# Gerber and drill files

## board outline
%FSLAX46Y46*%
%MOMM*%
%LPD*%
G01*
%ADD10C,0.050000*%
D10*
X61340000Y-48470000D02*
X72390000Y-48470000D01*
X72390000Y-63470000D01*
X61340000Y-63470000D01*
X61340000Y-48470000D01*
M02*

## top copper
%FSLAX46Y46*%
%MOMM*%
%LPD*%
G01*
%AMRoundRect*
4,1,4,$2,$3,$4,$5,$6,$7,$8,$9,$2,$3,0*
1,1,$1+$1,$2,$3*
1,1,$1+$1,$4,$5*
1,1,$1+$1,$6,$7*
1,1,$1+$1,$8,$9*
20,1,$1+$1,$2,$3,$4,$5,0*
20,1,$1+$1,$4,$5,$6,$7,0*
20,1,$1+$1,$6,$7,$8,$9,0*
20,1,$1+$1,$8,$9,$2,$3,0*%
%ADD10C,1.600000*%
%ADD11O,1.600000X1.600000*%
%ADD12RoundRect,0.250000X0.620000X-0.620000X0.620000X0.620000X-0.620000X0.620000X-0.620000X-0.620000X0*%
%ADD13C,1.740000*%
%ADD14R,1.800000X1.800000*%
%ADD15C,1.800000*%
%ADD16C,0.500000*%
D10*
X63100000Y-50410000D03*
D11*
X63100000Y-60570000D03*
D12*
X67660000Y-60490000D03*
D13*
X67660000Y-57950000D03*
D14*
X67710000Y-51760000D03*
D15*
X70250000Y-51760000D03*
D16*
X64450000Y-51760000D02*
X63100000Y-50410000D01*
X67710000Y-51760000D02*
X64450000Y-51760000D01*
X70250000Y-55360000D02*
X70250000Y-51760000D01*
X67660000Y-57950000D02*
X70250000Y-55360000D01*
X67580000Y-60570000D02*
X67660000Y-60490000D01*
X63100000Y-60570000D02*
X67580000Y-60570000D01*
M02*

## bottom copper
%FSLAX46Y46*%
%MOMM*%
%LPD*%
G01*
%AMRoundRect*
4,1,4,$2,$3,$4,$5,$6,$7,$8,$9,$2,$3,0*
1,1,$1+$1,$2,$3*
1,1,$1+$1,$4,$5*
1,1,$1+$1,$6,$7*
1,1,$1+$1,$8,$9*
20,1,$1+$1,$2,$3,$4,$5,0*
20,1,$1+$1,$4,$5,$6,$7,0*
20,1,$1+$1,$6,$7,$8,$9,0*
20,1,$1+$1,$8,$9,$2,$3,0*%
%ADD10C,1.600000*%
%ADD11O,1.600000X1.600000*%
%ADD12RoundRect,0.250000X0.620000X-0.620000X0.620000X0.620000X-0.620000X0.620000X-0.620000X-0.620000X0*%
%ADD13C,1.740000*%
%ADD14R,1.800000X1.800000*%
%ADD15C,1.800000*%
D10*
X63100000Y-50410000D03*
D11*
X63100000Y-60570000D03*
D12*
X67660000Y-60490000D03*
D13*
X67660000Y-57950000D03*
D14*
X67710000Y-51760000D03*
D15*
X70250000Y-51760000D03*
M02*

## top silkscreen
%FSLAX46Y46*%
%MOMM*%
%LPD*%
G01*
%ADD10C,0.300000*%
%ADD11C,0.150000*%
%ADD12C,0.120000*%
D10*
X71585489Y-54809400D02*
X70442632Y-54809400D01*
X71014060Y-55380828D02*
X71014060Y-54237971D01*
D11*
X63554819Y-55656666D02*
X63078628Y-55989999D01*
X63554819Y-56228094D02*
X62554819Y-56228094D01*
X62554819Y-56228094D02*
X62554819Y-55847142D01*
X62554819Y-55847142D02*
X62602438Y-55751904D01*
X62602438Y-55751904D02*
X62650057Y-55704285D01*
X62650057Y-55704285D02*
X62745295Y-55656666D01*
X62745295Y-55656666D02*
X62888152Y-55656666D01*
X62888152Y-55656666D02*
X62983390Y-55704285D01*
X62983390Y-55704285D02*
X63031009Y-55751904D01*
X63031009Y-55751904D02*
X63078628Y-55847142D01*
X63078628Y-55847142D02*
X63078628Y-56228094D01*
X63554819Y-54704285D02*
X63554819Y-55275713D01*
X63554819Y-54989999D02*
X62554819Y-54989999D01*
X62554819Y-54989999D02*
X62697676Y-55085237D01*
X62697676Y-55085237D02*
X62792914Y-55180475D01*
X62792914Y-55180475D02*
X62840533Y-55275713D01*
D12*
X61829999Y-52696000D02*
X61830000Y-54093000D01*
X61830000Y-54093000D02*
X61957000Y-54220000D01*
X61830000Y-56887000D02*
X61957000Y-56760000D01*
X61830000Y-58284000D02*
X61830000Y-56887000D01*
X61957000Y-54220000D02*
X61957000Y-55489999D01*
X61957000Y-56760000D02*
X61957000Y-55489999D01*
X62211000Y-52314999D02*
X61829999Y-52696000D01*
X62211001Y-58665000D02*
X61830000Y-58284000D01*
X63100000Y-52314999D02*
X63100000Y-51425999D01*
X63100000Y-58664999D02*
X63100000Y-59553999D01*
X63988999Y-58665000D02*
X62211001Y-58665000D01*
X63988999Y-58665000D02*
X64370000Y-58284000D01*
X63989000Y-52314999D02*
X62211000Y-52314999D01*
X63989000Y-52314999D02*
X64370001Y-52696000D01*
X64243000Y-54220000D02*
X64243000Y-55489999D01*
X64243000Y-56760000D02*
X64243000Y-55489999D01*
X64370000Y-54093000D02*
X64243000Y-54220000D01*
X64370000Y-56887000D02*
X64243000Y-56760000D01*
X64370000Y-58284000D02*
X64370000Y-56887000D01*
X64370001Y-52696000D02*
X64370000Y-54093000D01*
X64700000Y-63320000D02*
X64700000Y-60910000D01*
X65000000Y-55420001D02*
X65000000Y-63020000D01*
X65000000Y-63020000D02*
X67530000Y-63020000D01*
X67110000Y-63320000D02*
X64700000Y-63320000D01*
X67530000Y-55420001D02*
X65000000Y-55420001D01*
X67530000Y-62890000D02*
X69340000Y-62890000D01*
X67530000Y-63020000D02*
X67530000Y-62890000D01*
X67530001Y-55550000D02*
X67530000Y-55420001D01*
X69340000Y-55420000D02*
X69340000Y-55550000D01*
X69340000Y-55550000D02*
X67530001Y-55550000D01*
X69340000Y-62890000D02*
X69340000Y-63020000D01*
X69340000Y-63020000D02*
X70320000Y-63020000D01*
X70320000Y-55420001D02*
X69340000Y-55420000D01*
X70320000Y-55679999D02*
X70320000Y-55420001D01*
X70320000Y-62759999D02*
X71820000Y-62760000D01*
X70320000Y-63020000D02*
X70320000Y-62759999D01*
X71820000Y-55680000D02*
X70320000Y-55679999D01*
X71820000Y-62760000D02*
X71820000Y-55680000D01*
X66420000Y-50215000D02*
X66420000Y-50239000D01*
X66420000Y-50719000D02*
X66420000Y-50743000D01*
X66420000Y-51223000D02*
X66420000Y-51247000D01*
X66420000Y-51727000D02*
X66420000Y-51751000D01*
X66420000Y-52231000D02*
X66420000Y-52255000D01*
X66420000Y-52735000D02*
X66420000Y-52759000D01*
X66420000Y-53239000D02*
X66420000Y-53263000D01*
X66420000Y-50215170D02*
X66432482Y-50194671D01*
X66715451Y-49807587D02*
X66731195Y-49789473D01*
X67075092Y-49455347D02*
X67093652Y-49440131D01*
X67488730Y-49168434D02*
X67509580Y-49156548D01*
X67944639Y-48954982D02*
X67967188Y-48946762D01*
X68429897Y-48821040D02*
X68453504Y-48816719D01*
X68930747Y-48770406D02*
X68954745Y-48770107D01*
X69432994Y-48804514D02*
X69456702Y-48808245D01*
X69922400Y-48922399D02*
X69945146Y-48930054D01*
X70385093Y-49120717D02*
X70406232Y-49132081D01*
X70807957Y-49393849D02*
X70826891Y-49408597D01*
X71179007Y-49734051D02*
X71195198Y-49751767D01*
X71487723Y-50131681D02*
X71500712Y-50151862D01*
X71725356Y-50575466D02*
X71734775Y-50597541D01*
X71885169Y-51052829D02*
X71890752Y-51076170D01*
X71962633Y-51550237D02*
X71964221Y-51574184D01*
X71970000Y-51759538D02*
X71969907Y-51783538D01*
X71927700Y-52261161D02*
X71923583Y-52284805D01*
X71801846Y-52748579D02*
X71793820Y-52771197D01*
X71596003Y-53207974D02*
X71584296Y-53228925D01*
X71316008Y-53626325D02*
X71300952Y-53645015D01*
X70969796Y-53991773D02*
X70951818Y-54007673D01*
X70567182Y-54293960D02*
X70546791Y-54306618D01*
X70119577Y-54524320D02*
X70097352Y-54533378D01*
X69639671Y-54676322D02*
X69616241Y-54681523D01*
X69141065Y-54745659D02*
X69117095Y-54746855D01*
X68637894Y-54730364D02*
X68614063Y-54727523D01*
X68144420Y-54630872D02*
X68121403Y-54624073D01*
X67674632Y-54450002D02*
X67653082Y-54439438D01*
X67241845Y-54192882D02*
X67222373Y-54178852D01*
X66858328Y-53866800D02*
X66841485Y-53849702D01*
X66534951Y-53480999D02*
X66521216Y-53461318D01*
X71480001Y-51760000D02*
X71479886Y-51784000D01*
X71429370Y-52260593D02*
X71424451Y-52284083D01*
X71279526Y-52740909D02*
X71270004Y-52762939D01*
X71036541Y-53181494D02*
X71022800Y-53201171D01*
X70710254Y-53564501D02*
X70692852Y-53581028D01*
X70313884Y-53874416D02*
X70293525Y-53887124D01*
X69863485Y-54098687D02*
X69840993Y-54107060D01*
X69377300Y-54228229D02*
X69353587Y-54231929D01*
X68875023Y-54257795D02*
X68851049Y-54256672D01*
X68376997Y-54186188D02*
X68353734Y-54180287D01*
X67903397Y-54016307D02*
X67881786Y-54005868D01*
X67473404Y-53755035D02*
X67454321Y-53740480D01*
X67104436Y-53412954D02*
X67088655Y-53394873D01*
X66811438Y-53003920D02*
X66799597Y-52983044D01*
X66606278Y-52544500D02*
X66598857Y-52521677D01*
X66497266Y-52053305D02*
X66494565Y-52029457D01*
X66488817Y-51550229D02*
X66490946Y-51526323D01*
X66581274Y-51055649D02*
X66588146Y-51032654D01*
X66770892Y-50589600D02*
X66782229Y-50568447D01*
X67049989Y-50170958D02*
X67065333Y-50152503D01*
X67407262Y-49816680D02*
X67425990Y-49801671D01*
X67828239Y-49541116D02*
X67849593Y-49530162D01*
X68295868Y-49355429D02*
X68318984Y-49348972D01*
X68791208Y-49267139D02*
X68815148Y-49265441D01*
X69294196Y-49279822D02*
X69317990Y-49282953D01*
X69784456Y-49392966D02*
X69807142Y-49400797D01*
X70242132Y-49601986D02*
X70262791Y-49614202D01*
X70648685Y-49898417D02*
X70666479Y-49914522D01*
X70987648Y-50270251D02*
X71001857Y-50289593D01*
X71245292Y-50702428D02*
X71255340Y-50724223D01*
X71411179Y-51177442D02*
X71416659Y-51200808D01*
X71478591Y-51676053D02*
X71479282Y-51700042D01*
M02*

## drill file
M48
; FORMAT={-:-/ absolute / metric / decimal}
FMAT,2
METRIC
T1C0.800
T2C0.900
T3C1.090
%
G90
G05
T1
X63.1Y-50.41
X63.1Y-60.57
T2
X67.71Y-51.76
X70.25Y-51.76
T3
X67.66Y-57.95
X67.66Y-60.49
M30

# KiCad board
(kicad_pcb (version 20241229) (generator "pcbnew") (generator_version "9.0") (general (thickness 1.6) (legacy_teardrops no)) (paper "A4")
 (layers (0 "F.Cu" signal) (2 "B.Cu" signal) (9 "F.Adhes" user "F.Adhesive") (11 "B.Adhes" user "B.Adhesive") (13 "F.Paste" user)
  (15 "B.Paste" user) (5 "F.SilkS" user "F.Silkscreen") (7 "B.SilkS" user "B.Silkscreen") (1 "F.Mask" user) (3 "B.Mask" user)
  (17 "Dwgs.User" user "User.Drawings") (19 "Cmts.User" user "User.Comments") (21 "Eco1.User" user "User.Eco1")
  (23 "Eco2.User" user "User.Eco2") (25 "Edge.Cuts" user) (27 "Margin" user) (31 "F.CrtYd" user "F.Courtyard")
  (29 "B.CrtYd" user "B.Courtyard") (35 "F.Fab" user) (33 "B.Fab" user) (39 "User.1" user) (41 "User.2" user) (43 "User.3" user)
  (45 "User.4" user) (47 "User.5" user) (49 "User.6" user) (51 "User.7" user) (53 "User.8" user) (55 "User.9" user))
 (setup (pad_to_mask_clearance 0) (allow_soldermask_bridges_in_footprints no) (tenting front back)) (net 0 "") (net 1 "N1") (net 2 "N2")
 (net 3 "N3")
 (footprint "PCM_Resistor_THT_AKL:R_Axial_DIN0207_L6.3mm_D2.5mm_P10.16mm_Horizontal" (layer "F.Cu") (at 63.1 50.41 -90)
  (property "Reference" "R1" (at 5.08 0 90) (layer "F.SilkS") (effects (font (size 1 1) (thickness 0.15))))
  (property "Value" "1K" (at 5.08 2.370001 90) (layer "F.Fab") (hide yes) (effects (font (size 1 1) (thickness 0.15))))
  (fp_line (start 2.286 1.270001) (end 3.683 1.27) (stroke (width 0.12) (type solid)) (layer "F.SilkS"))
  (fp_line (start 3.683 1.27) (end 3.81 1.143) (stroke (width 0.12) (type solid)) (layer "F.SilkS"))
  (fp_line (start 6.477 1.27) (end 6.35 1.143) (stroke (width 0.12) (type solid)) (layer "F.SilkS"))
  (fp_line (start 7.874 1.27) (end 6.477 1.27) (stroke (width 0.12) (type solid)) (layer "F.SilkS"))
  (fp_line (start 3.81 1.143) (end 5.079999 1.143) (stroke (width 0.12) (type solid)) (layer "F.SilkS"))
  (fp_line (start 6.35 1.143) (end 5.079999 1.143) (stroke (width 0.12) (type solid)) (layer "F.SilkS"))
  (fp_line (start 1.904999 0.889) (end 2.286 1.270001) (stroke (width 0.12) (type solid)) (layer "F.SilkS"))
  (fp_line (start 8.255 0.888999) (end 7.874 1.27) (stroke (width 0.12) (type solid)) (layer "F.SilkS"))
  (fp_line (start 1.904999 0) (end 1.015999 0) (stroke (width 0.12) (type solid)) (layer "F.SilkS"))
  (fp_line (start 8.254999 0) (end 9.143999 0) (stroke (width 0.12) (type solid)) (layer "F.SilkS"))
  (fp_line (start 8.255 -0.888999) (end 8.255 0.888999) (stroke (width 0.12) (type solid)) (layer "F.SilkS"))
  (fp_line (start 8.255 -0.888999) (end 7.874 -1.27) (stroke (width 0.12) (type solid)) (layer "F.SilkS"))
  (fp_line (start 1.904999 -0.889) (end 1.904999 0.889) (stroke (width 0.12) (type solid)) (layer "F.SilkS"))
  (fp_line (start 1.904999 -0.889) (end 2.286 -1.270001) (stroke (width 0.12) (type solid)) (layer "F.SilkS"))
  (fp_line (start 3.81 -1.143) (end 5.079999 -1.143) (stroke (width 0.12) (type solid)) (layer "F.SilkS"))
  (fp_line (start 6.35 -1.143) (end 5.079999 -1.143) (stroke (width 0.12) (type solid)) (layer "F.SilkS"))
  (fp_line (start 3.683 -1.27) (end 3.81 -1.143) (stroke (width 0.12) (type solid)) (layer "F.SilkS"))
  (fp_line (start 6.477 -1.27) (end 6.35 -1.143) (stroke (width 0.12) (type solid)) (layer "F.SilkS"))
  (fp_line (start 7.874 -1.27) (end 6.477 -1.27) (stroke (width 0.12) (type solid)) (layer "F.SilkS"))
  (fp_line (start 2.286 -1.270001) (end 3.683 -1.27) (stroke (width 0.12) (type solid)) (layer "F.SilkS"))
  (pad "1" thru_hole circle (at 0 0 270) (size 1.6 1.6) (drill 0.8) (layers "*.Cu" "*.Mask") (remove_unused_layers no) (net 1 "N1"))
  (pad "2" thru_hole oval (at 10.16 0 270) (size 1.6 1.6) (drill 0.8) (layers "*.Cu" "*.Mask") (remove_unused_layers no) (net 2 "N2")))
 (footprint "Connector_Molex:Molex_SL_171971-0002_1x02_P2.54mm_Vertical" (layer "F.Cu") (at 67.66 60.49 90)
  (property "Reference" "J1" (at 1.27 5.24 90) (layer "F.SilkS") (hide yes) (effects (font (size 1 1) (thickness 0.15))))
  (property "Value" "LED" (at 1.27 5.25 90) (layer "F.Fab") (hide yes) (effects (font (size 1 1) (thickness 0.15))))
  (fp_line (start -2.83 -2.96) (end -0.42 -2.96) (stroke (width 0.12) (type solid)) (layer "F.SilkS"))
  (fp_line (start 5.069999 -2.66) (end -2.53 -2.66) (stroke (width 0.12) (type solid)) (layer "F.SilkS"))
  (fp_line (start -2.53 -2.66) (end -2.53 -0.13) (stroke (width 0.12) (type solid)) (layer "F.SilkS"))
  (fp_line (start -2.83 -0.55) (end -2.83 -2.96) (stroke (width 0.12) (type solid)) (layer "F.SilkS"))
  (fp_line (start 5.069999 -0.13) (end 5.069999 -2.66) (stroke (width 0.12) (type solid)) (layer "F.SilkS"))
  (fp_line (start -2.4 -0.13) (end -2.4 1.68) (stroke (width 0.12) (type solid)) (layer "F.SilkS"))
  (fp_line (start -2.53 -0.13) (end -2.4 -0.13) (stroke (width 0.12) (type solid)) (layer "F.SilkS"))
  (fp_line (start 4.94 -0.129999) (end 5.069999 -0.13) (stroke (width 0.12) (type solid)) (layer "F.SilkS"))
  (fp_line (start 5.07 1.68) (end 4.94 1.68) (stroke (width 0.12) (type solid)) (layer "F.SilkS"))
  (fp_line (start 4.94 1.68) (end 4.94 -0.129999) (stroke (width 0.12) (type solid)) (layer "F.SilkS"))
  (fp_line (start -2.4 1.68) (end -2.53 1.68) (stroke (width 0.12) (type solid)) (layer "F.SilkS"))
  (fp_line (start -2.53 1.68) (end -2.53 2.66) (stroke (width 0.12) (type solid)) (layer "F.SilkS"))
  (fp_line (start 5.069999 2.66) (end 5.07 1.68) (stroke (width 0.12) (type solid)) (layer "F.SilkS"))
  (fp_line (start 4.810001 2.66) (end 5.069999 2.66) (stroke (width 0.12) (type solid)) (layer "F.SilkS"))
  (fp_line (start -2.269999 2.66) (end -2.27 4.16) (stroke (width 0.12) (type solid)) (layer "F.SilkS"))
  (fp_line (start -2.53 2.66) (end -2.269999 2.66) (stroke (width 0.12) (type solid)) (layer "F.SilkS"))
  (fp_line (start 4.81 4.16) (end 4.810001 2.66) (stroke (width 0.12) (type solid)) (layer "F.SilkS"))
  (fp_line (start -2.27 4.16) (end 4.81 4.16) (stroke (width 0.12) (type solid)) (layer "F.SilkS"))
  (pad "1" thru_hole roundrect (at 0 0 90) (size 1.74 1.74) (drill 1.09) (layers "*.Cu" "*.Mask") (remove_unused_layers no)
   (roundrect_rratio 0.143678) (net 2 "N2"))
  (pad "2" thru_hole circle (at 2.54 0 90) (size 1.74 1.74) (drill 1.09) (layers "*.Cu" "*.Mask") (remove_unused_layers no) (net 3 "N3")))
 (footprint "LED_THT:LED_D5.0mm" (layer "B.Cu") (at 67.71 51.76)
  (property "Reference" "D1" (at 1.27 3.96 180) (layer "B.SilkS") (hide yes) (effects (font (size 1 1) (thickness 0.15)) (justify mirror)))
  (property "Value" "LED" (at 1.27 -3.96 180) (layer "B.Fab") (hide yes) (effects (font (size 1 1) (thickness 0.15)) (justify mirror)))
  (fp_line (start -1.29 -1.545) (end -1.29 1.545) (stroke (width 0.12) (type dot)) (layer "F.SilkS"))
  (fp_arc (start -1.29 -1.54483) (mid 2.072002 -2.880433) (end 4.26 0.000462) (stroke (width 0.12) (type dot)) (layer "F.SilkS"))
  (fp_arc (start 4.26 -0.000462) (mid 2.072002 2.880435) (end -1.29 1.54483) (stroke (width 0.12) (type dot)) (layer "F.SilkS"))
  (fp_circle (center 1.270001 0) (end 3.770001 0) (stroke (width 0.12) (type dot)) (fill no) (layer "F.SilkS"))
  (pad "1" thru_hole rect (at 0 0) (size 1.8 1.8) (drill 0.9) (layers "*.Cu" "*.Mask") (remove_unused_layers no) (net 1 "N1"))
  (pad "2" thru_hole circle (at 2.54 0) (size 1.8 1.8) (drill 0.9) (layers "*.Cu" "*.Mask") (remove_unused_layers no) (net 3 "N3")))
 (gr_rect (start 61.34 48.47) (end 72.39 63.47) (stroke (width 0.05) (type default)) (fill no) (layer "Edge.Cuts"))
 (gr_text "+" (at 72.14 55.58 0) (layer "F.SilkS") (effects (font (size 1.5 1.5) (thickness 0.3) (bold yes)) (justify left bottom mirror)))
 (segment (start 64.45 51.76) (end 63.1 50.41) (width 0.5) (layer "F.Cu") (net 1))
 (segment (start 67.71 51.76) (end 64.45 51.76) (width 0.5) (layer "F.Cu") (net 1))
 (segment (start 70.25 55.36) (end 70.25 51.76) (width 0.5) (layer "F.Cu") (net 3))
 (segment (start 67.66 57.95) (end 70.25 55.36) (width 0.5) (layer "F.Cu") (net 3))
 (segment (start 67.58 60.57) (end 67.66 60.49) (width 0.5) (layer "F.Cu") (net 2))
 (segment (start 63.1 60.57) (end 67.58 60.57) (width 0.5) (layer "F.Cu") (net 2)))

